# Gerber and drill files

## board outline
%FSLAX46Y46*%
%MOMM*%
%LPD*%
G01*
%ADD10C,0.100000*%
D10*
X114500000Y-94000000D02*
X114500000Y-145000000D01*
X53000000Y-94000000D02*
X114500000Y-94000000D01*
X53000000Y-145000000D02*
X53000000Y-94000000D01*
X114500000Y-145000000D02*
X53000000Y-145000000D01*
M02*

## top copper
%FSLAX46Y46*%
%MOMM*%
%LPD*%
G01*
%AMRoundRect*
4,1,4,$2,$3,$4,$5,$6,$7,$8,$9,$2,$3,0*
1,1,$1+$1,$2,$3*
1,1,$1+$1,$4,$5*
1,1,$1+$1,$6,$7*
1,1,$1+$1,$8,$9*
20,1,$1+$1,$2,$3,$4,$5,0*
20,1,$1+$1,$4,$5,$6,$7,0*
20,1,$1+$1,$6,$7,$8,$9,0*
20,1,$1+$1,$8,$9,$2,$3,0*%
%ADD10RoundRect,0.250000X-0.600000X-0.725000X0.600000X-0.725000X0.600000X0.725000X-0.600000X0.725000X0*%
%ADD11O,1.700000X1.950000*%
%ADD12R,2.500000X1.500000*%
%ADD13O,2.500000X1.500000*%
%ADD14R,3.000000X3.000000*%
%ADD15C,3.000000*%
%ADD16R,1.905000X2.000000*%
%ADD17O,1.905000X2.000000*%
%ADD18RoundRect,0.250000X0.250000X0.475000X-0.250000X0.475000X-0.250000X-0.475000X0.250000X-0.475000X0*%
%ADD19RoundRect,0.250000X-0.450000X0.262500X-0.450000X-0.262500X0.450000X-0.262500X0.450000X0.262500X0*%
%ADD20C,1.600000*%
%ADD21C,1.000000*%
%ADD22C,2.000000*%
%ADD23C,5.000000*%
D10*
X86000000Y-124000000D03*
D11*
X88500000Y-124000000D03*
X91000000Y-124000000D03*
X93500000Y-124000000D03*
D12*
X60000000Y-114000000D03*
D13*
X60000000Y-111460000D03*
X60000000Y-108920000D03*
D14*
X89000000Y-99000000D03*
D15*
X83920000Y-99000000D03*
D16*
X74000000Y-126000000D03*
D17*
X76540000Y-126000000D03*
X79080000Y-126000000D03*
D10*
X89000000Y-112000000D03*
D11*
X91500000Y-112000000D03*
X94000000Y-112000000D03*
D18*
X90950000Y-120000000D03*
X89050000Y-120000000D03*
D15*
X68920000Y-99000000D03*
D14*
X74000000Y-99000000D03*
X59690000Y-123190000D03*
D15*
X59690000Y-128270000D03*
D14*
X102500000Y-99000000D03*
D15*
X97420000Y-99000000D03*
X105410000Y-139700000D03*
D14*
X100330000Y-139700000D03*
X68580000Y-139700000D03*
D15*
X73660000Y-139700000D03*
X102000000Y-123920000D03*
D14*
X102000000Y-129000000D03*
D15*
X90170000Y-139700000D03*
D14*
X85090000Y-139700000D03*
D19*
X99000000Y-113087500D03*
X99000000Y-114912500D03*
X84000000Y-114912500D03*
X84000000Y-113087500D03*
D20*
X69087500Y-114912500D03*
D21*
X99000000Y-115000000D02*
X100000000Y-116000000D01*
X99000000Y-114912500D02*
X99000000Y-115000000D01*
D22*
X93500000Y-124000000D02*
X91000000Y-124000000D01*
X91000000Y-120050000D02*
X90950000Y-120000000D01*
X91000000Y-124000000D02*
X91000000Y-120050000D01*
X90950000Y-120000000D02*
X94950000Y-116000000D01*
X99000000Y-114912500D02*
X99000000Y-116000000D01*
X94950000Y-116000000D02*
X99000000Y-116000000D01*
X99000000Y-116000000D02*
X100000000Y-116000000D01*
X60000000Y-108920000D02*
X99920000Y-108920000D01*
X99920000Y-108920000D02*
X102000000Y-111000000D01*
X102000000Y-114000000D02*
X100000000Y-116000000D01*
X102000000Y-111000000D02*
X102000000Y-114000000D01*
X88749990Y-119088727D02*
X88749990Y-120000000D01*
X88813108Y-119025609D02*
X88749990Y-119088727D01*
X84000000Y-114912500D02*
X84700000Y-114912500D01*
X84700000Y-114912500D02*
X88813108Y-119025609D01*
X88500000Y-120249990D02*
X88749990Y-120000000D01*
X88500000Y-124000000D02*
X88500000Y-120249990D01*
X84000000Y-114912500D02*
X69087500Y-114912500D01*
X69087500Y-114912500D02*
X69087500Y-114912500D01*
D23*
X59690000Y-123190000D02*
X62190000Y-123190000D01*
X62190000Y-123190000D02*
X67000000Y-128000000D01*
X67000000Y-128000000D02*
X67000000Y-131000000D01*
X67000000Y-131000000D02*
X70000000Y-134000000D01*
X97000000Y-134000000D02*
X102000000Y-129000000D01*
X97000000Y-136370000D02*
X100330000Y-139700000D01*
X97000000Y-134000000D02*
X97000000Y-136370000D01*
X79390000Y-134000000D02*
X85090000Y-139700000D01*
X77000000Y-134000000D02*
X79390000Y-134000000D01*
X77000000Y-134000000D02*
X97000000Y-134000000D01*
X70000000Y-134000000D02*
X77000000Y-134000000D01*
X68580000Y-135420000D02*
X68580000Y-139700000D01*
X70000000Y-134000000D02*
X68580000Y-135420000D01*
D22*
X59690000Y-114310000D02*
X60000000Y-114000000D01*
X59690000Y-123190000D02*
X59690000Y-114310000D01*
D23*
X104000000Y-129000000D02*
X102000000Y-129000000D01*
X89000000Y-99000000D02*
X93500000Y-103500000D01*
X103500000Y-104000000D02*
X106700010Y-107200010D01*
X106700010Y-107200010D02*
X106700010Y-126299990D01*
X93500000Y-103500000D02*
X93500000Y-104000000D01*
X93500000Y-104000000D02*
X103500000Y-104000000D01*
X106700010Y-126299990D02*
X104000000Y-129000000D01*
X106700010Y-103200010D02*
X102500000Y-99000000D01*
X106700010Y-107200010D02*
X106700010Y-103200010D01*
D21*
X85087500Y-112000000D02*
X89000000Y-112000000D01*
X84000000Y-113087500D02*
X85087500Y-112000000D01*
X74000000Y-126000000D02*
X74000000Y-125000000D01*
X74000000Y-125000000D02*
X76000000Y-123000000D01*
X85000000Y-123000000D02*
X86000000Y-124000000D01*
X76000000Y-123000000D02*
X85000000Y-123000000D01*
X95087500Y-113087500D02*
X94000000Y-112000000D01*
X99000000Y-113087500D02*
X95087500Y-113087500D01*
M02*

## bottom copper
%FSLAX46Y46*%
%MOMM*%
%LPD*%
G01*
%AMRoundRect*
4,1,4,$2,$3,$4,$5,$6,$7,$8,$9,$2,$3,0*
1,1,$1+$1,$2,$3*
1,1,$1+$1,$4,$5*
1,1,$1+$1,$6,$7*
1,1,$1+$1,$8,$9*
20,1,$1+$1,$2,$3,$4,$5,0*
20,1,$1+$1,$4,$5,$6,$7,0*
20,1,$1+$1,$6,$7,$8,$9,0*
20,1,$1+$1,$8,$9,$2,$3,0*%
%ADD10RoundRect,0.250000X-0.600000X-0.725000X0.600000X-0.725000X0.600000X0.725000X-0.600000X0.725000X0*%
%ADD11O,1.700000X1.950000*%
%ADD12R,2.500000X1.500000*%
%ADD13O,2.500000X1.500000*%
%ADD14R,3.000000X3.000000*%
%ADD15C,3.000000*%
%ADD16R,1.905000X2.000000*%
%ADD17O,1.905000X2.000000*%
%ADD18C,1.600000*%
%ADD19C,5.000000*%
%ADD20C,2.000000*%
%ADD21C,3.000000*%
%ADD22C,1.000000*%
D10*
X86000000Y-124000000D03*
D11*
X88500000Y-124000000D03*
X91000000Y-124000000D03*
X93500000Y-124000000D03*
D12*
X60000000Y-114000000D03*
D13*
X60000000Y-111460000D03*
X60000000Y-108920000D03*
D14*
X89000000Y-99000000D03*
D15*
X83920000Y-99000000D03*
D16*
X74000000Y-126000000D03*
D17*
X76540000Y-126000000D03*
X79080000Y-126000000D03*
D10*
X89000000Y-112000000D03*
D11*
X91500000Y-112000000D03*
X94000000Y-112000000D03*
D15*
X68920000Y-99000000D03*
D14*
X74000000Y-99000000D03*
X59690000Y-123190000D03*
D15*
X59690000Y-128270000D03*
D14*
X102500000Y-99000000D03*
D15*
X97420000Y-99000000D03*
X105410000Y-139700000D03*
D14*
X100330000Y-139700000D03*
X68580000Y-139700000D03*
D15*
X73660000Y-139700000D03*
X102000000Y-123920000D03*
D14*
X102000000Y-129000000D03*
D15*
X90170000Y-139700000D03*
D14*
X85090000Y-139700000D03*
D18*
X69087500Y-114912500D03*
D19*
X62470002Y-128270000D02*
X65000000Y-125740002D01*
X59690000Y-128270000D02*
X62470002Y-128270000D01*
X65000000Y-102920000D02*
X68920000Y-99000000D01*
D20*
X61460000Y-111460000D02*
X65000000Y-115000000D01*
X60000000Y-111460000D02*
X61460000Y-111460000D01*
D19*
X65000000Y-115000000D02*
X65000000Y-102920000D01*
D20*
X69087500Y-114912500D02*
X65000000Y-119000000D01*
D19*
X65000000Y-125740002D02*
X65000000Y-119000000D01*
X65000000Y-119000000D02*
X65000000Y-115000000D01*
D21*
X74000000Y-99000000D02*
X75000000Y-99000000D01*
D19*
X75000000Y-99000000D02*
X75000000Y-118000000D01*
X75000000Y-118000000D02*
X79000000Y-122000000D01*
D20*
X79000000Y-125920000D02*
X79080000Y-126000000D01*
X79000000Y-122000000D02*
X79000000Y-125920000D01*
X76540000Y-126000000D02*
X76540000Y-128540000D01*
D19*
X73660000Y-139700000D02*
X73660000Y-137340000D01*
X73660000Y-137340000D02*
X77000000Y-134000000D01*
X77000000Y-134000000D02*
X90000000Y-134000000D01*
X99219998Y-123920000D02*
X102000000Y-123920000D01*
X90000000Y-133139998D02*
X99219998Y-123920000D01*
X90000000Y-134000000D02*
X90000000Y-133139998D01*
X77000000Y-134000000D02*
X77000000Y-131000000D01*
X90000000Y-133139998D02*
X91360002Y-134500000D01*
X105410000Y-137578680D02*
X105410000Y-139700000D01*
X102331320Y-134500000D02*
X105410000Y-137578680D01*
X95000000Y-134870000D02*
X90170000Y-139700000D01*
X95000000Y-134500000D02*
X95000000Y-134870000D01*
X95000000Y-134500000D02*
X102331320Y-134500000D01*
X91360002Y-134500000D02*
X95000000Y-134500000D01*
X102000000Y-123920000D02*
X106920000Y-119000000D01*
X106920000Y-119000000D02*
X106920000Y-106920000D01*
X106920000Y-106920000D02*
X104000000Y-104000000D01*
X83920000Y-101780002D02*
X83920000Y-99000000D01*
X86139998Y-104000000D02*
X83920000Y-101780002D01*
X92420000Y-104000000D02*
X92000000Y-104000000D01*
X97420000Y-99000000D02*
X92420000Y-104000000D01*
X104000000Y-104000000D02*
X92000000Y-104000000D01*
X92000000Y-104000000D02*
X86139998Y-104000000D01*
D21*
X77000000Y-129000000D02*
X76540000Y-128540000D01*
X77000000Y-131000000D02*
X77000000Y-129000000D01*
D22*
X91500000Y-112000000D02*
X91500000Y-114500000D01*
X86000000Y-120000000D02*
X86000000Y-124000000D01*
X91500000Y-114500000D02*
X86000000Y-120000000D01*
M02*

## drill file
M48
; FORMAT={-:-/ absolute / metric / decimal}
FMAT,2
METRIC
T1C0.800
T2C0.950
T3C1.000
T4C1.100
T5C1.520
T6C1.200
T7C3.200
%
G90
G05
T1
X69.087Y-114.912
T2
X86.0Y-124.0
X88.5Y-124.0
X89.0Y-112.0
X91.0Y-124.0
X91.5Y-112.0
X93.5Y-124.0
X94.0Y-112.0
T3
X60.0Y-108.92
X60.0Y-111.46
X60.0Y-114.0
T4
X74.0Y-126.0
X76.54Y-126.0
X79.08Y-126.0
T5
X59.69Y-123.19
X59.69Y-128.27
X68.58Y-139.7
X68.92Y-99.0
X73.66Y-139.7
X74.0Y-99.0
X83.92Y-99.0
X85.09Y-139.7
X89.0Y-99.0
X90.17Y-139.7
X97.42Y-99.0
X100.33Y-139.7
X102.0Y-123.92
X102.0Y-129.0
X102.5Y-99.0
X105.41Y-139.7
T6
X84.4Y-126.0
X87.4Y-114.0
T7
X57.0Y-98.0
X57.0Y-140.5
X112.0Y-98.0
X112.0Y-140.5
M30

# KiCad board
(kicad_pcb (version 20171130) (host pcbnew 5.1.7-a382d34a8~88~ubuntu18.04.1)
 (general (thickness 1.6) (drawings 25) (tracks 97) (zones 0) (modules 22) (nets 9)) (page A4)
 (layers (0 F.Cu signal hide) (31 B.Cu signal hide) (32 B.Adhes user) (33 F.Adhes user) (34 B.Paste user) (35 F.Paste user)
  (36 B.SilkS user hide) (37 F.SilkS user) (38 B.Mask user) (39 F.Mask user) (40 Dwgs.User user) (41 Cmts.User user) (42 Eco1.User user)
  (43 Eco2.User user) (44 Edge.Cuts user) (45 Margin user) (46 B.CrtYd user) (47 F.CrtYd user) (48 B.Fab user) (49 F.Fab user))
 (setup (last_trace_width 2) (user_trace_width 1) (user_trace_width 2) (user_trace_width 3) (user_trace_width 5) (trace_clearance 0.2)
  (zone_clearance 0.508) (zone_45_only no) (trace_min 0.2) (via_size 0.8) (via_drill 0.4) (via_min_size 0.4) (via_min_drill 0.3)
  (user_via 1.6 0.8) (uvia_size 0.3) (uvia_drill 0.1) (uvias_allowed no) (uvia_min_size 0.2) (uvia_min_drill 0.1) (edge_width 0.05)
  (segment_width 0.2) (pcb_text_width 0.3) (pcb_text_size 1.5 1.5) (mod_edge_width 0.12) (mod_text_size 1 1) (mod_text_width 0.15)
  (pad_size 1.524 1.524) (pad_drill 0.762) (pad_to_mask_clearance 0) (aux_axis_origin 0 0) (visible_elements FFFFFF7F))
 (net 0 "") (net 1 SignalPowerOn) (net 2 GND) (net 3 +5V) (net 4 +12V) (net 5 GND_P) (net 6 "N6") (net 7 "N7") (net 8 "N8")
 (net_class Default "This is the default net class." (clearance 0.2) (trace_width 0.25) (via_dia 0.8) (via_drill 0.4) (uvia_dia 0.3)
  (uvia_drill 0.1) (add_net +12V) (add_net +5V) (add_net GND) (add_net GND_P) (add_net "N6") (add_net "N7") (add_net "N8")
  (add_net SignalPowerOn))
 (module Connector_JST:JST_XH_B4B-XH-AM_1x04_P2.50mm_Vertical (layer F.Cu) (at 86 124)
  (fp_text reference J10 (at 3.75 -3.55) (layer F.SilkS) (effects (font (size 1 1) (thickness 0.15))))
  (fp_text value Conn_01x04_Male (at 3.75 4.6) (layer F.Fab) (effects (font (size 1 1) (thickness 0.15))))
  (pad 1 thru_hole roundrect (at 0 0) (size 1.7 1.95) (drill 0.95) (layers *.Cu *.Mask) (roundrect_rratio 0.147059) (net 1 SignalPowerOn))
  (pad 2 thru_hole oval (at 2.5 0) (size 1.7 1.95) (drill 0.95) (layers *.Cu *.Mask) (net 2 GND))
  (pad 3 thru_hole oval (at 5 0) (size 1.7 1.95) (drill 0.95) (layers *.Cu *.Mask) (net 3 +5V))
  (pad 4 thru_hole oval (at 7.5 0) (size 1.7 1.95) (drill 0.95) (layers *.Cu *.Mask) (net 3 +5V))
  (pad "" np_thru_hole circle (at -1.6 2) (size 1.2 1.2) (drill 1.2) (layers *.Cu *.Mask)))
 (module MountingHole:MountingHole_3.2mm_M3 (layer F.Cu) (at 57 98)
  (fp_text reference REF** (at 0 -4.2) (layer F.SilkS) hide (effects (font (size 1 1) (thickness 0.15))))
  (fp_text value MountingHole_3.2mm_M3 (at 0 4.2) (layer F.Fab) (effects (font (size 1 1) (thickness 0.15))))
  (pad 1 np_thru_hole circle (at 0 0) (size 3.2 3.2) (drill 3.2) (layers *.Cu *.Mask)))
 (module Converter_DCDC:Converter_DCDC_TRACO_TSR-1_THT (layer F.Cu) (at 60 114 90)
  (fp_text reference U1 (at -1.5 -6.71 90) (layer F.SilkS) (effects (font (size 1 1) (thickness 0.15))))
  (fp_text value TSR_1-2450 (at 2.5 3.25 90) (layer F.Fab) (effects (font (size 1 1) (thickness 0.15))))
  (pad 1 thru_hole rect (at 0 0 90) (size 1.5 2.5) (drill 1) (layers *.Cu *.Mask) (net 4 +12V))
  (pad 2 thru_hole oval (at 2.54 0 90) (size 1.5 2.5) (drill 1) (layers *.Cu *.Mask) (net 2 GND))
  (pad 3 thru_hole oval (at 5.08 0 90) (size 1.5 2.5) (drill 1) (layers *.Cu *.Mask) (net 3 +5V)))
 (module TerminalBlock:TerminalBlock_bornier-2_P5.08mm (layer F.Cu) (at 89 99 180)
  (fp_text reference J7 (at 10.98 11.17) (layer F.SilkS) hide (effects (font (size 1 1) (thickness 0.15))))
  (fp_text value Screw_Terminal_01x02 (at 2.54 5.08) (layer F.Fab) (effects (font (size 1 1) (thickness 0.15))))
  (pad 1 thru_hole rect (at 0 0 180) (size 3 3) (drill 1.52) (layers *.Cu *.Mask) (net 4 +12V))
  (pad 2 thru_hole circle (at 5.08 0 180) (size 3 3) (drill 1.52) (layers *.Cu *.Mask) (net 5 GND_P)))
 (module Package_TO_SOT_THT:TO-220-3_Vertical (layer F.Cu) (at 74 126)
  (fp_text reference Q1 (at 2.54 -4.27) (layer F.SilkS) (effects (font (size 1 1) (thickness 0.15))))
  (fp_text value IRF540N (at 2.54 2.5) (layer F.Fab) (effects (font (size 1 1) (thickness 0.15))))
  (pad 1 thru_hole rect (at 0 0) (size 1.905 2) (drill 1.1) (layers *.Cu *.Mask) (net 1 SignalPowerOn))
  (pad 2 thru_hole oval (at 2.54 0) (size 1.905 2) (drill 1.1) (layers *.Cu *.Mask) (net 5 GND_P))
  (pad 3 thru_hole oval (at 5.08 0) (size 1.905 2) (drill 1.1) (layers *.Cu *.Mask) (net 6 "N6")))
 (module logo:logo (layer B.Cu) (at 78 111.5)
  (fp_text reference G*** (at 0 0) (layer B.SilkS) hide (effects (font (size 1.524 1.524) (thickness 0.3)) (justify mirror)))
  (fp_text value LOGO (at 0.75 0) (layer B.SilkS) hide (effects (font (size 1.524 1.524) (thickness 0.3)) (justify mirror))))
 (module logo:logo (layer F.Cu) (at 69 -16)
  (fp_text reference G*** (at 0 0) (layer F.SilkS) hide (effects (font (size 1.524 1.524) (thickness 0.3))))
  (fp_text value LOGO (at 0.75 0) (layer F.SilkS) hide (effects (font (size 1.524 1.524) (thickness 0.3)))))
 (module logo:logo (layer F.Cu) (at 94 104)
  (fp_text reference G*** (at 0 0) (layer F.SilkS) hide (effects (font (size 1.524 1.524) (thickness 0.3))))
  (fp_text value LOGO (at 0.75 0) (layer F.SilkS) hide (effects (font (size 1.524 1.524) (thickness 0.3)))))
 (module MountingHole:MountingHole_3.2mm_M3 (layer F.Cu) (at 57 140.5)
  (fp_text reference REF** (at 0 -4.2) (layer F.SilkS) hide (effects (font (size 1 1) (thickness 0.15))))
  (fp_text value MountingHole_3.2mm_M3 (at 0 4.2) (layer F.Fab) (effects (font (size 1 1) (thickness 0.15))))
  (pad 1 np_thru_hole circle (at 0 0) (size 3.2 3.2) (drill 3.2) (layers *.Cu *.Mask)))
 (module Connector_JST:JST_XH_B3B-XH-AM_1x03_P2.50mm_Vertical (layer F.Cu) (at 89 112)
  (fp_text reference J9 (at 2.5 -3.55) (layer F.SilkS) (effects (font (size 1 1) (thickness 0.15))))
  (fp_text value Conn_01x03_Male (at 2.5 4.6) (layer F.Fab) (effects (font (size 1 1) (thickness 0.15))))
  (pad 1 thru_hole roundrect (at 0 0) (size 1.7 1.95) (drill 0.95) (layers *.Cu *.Mask) (roundrect_rratio 0.147059) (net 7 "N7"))
  (pad 2 thru_hole oval (at 2.5 0) (size 1.7 1.95) (drill 0.95) (layers *.Cu *.Mask) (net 1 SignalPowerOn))
  (pad 3 thru_hole oval (at 5 0) (size 1.7 1.95) (drill 0.95) (layers *.Cu *.Mask) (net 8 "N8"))
  (pad "" np_thru_hole circle (at -1.6 2) (size 1.2 1.2) (drill 1.2) (layers *.Cu *.Mask)))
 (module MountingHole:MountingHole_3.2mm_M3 (layer F.Cu) (at 112 98)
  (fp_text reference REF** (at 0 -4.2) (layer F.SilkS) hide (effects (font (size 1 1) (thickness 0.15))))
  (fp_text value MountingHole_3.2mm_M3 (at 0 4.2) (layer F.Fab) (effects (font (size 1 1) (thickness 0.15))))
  (pad 1 np_thru_hole circle (at 0 0) (size 3.2 3.2) (drill 3.2) (layers *.Cu *.Mask)))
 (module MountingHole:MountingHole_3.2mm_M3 (layer F.Cu) (at 112 140.5)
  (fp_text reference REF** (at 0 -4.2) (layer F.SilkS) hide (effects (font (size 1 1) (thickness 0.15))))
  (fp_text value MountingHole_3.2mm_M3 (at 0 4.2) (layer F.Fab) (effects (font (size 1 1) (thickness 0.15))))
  (pad 1 np_thru_hole circle (at 0 0) (size 3.2 3.2) (drill 3.2) (layers *.Cu *.Mask)))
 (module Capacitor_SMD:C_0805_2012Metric (layer F.Cu) (at 90 120 180)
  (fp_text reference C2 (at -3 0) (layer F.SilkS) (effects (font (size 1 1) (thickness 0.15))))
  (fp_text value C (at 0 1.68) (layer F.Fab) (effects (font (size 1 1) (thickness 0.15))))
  (pad 1 smd roundrect (at -0.95 0 180) (size 1 1.45) (layers F.Cu F.Paste F.Mask) (roundrect_rratio 0.25) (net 3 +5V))
  (pad 2 smd roundrect (at 0.95 0 180) (size 1 1.45) (layers F.Cu F.Paste F.Mask) (roundrect_rratio 0.25) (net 2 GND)))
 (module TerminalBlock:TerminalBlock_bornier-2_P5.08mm (layer F.Cu) (at 74 99 180)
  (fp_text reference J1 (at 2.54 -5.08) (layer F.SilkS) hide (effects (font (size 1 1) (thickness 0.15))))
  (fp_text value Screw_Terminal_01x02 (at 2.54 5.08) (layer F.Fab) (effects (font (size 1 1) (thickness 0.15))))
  (pad 2 thru_hole circle (at 5.08 0 180) (size 3 3) (drill 1.52) (layers *.Cu *.Mask) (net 2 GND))
  (pad 1 thru_hole rect (at 0 0 180) (size 3 3) (drill 1.52) (layers *.Cu *.Mask) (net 6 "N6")))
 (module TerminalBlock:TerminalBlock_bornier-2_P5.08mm (layer F.Cu) (at 59.69 123.19 270)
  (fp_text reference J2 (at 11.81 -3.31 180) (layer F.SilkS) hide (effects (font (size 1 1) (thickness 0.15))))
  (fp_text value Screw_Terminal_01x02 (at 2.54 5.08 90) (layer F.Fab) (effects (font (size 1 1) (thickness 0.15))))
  (pad 1 thru_hole rect (at 0 0 270) (size 3 3) (drill 1.52) (layers *.Cu *.Mask) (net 4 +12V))
  (pad 2 thru_hole circle (at 5.08 0 270) (size 3 3) (drill 1.52) (layers *.Cu *.Mask) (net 2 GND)))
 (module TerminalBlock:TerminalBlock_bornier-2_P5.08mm (layer F.Cu) (at 102.5 99 180)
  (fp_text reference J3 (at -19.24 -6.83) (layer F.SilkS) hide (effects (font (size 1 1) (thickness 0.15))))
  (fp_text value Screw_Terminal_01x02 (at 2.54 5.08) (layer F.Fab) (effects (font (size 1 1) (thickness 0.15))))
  (pad 1 thru_hole rect (at 0 0 180) (size 3 3) (drill 1.52) (layers *.Cu *.Mask) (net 4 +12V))
  (pad 2 thru_hole circle (at 5.08 0 180) (size 3 3) (drill 1.52) (layers *.Cu *.Mask) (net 5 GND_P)))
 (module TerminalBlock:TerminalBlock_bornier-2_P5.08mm (layer F.Cu) (at 100.33 139.7)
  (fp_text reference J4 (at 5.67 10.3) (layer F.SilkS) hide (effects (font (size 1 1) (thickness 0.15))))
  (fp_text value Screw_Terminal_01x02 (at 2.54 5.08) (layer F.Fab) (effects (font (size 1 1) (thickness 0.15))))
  (pad 2 thru_hole circle (at 5.08 0) (size 3 3) (drill 1.52) (layers *.Cu *.Mask) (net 5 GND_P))
  (pad 1 thru_hole rect (at 0 0) (size 3 3) (drill 1.52) (layers *.Cu *.Mask) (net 4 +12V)))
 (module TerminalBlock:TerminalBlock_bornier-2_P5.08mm (layer F.Cu) (at 68.58 139.7)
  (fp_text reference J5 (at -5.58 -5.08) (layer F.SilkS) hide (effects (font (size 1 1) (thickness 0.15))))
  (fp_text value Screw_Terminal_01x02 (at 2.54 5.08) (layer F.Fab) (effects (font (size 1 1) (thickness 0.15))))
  (pad 1 thru_hole rect (at 0 0) (size 3 3) (drill 1.52) (layers *.Cu *.Mask) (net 4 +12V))
  (pad 2 thru_hole circle (at 5.08 0) (size 3 3) (drill 1.52) (layers *.Cu *.Mask) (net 5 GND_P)))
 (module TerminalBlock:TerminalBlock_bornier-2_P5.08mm (layer F.Cu) (at 102 129 90)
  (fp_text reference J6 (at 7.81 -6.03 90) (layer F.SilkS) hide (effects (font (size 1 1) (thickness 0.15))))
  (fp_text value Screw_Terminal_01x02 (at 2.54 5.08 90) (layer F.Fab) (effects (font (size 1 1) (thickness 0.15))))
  (pad 2 thru_hole circle (at 5.08 0 90) (size 3 3) (drill 1.52) (layers *.Cu *.Mask) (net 5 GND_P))
  (pad 1 thru_hole rect (at 0 0 90) (size 3 3) (drill 1.52) (layers *.Cu *.Mask) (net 4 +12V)))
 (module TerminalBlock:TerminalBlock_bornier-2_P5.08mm (layer F.Cu) (at 85.09 139.7)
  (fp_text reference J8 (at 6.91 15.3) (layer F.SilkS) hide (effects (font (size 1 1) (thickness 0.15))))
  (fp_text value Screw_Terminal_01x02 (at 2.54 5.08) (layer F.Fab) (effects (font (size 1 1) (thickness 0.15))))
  (pad 2 thru_hole circle (at 5.08 0) (size 3 3) (drill 1.52) (layers *.Cu *.Mask) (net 5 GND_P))
  (pad 1 thru_hole rect (at 0 0) (size 3 3) (drill 1.52) (layers *.Cu *.Mask) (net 4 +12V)))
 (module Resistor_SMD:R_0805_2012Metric (layer F.Cu) (at 99 114 270)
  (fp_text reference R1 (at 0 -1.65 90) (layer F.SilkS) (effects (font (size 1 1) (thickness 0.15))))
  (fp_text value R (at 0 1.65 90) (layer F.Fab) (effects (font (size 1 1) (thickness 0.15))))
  (pad 1 smd roundrect (at -0.9125 0 270) (size 1.025 1.4) (layers F.Cu F.Paste F.Mask) (roundrect_rratio 0.243902) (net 8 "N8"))
  (pad 2 smd roundrect (at 0.9125 0 270) (size 1.025 1.4) (layers F.Cu F.Paste F.Mask) (roundrect_rratio 0.243902) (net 3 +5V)))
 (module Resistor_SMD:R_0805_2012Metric (layer F.Cu) (at 84 114 270)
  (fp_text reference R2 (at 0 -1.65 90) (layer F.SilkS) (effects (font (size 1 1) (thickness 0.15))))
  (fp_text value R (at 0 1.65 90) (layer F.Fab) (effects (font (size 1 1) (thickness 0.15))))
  (pad 2 smd roundrect (at 0.9125 0 270) (size 1.025 1.4) (layers F.Cu F.Paste F.Mask) (roundrect_rratio 0.243902) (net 2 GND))
  (pad 1 smd roundrect (at -0.9125 0 270) (size 1.025 1.4) (layers F.Cu F.Paste F.Mask) (roundrect_rratio 0.243902) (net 7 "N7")))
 (gr_line (start 114.5 94) (end 114.5 145) (layer Edge.Cuts) (width 0.1))
 (gr_line (start 53 94) (end 114.5 94) (layer Edge.Cuts) (width 0.1))
 (gr_line (start 53 145) (end 53 94) (layer Edge.Cuts) (width 0.1))
 (gr_line (start 114.5 145) (end 53 145) (layer Edge.Cuts) (width 0.1))
 (segment (start 99 115) (end 100 116) (width 1) (layer F.Cu) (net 3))
 (segment (start 99 114.9125) (end 99 115) (width 1) (layer F.Cu) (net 3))
 (segment (start 93.5 124) (end 91 124) (width 2) (layer F.Cu) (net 3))
 (segment (start 91 120.05) (end 90.95 120) (width 2) (layer F.Cu) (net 3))
 (segment (start 91 124) (end 91 120.05) (width 2) (layer F.Cu) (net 3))
 (segment (start 90.95 120) (end 94.95 116) (width 2) (layer F.Cu) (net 3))
 (segment (start 99 114.9125) (end 99 116) (width 2) (layer F.Cu) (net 3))
 (segment (start 94.95 116) (end 99 116) (width 2) (layer F.Cu) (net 3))
 (segment (start 99 116) (end 100 116) (width 2) (layer F.Cu) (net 3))
 (segment (start 60 108.92) (end 99.92 108.92) (width 2) (layer F.Cu) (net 3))
 (segment (start 99.92 108.92) (end 102 111) (width 2) (layer F.Cu) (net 3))
 (segment (start 102 114) (end 100 116) (width 2) (layer F.Cu) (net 3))
 (segment (start 102 111) (end 102 114) (width 2) (layer F.Cu) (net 3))
 (segment (start 62.470002 128.27) (end 65 125.740002) (width 5) (layer B.Cu) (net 2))
 (segment (start 59.69 128.27) (end 62.470002 128.27) (width 5) (layer B.Cu) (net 2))
 (segment (start 65 102.92) (end 68.92 99) (width 5) (layer B.Cu) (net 2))
 (segment (start 61.46 111.46) (end 65 115) (width 2) (layer B.Cu) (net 2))
 (segment (start 60 111.46) (end 61.46 111.46) (width 2) (layer B.Cu) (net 2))
 (segment (start 65 115) (end 65 102.92) (width 5) (layer B.Cu) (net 2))
 (segment (start 88.74999 119.088727) (end 88.74999 120) (width 2) (layer F.Cu) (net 2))
 (segment (start 88.813108 119.025609) (end 88.74999 119.088727) (width 2) (layer F.Cu) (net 2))
 (segment (start 84 114.9125) (end 84.7 114.9125) (width 2) (layer F.Cu) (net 2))
 (segment (start 84.7 114.9125) (end 88.813108 119.025609) (width 2) (layer F.Cu) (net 2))
 (segment (start 88.5 120.24999) (end 88.74999 120) (width 2) (layer F.Cu) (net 2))
 (segment (start 88.5 124) (end 88.5 120.24999) (width 2) (layer F.Cu) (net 2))
 (segment (start 84 114.9125) (end 69.0875 114.9125) (width 2) (layer F.Cu) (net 2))
 (segment (start 69.0875 114.9125) (end 69.0875 114.9125) (width 2) (layer F.Cu) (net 2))
 (via (at 69.0875 114.9125) (size 1.6) (drill 0.8) (layers F.Cu B.Cu) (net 2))
 (segment (start 69.0875 114.9125) (end 65 119) (width 2) (layer B.Cu) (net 2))
 (segment (start 65 125.740002) (end 65 119) (width 5) (layer B.Cu) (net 2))
 (segment (start 65 119) (end 65 115) (width 5) (layer B.Cu) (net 2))
 (segment (start 74 99) (end 75 99) (width 3) (layer B.Cu) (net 6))
 (segment (start 75 99) (end 75 118) (width 5) (layer B.Cu) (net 6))
 (segment (start 75 118) (end 79 122) (width 5) (layer B.Cu) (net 6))
 (segment (start 79 125.92) (end 79.08 126) (width 2) (layer B.Cu) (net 6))
 (segment (start 79 122) (end 79 125.92) (width 2) (layer B.Cu) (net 6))
 (segment (start 59.69 123.19) (end 62.19 123.19) (width 5) (layer F.Cu) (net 4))
 (segment (start 62.19 123.19) (end 67 128) (width 5) (layer F.Cu) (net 4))
 (segment (start 67 128) (end 67 131) (width 5) (layer F.Cu) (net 4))
 (segment (start 67 131) (end 70 134) (width 5) (layer F.Cu) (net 4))
 (segment (start 97 134) (end 102 129) (width 5) (layer F.Cu) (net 4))
 (segment (start 97 136.37) (end 100.33 139.7) (width 5) (layer F.Cu) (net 4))
 (segment (start 97 134) (end 97 136.37) (width 5) (layer F.Cu) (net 4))
 (segment (start 79.39 134) (end 85.09 139.7) (width 5) (layer F.Cu) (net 4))
 (segment (start 77 134) (end 79.39 134) (width 5) (layer F.Cu) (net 4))
 (segment (start 77 134) (end 97 134) (width 5) (layer F.Cu) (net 4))
 (segment (start 70 134) (end 77 134) (width 5) (layer F.Cu) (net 4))
 (segment (start 68.58 135.42) (end 68.58 139.7) (width 5) (layer F.Cu) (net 4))
 (segment (start 70 134) (end 68.58 135.42) (width 5) (layer F.Cu) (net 4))
 (segment (start 59.69 114.31) (end 60 114) (width 2) (layer F.Cu) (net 4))
 (segment (start 59.69 123.19) (end 59.69 114.31) (width 2) (layer F.Cu) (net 4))
 (segment (start 104 129) (end 102 129) (width 5) (layer F.Cu) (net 4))
 (segment (start 89 99) (end 93.5 103.5) (width 5) (layer F.Cu) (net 4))
 (segment (start 103.5 104) (end 106.70001 107.20001) (width 5) (layer F.Cu) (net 4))
 (segment (start 106.70001 107.20001) (end 106.70001 126.29999) (width 5) (layer F.Cu) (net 4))
 (segment (start 93.5 103.5) (end 93.5 104) (width 5) (layer F.Cu) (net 4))
 (segment (start 93.5 104) (end 103.5 104) (width 5) (layer F.Cu) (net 4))
 (segment (start 106.70001 126.29999) (end 104 129) (width 5) (layer F.Cu) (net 4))
 (segment (start 106.70001 103.20001) (end 102.5 99) (width 5) (layer F.Cu) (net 4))
 (segment (start 106.70001 107.20001) (end 106.70001 103.20001) (width 5) (layer F.Cu) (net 4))
 (segment (start 76.54 126) (end 76.54 128.54) (width 2) (layer B.Cu) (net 5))
 (segment (start 73.66 139.7) (end 73.66 137.34) (width 5) (layer B.Cu) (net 5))
 (segment (start 73.66 137.34) (end 77 134) (width 5) (layer B.Cu) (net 5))
 (segment (start 77 134) (end 90 134) (width 5) (layer B.Cu) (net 5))
 (segment (start 99.219998 123.92) (end 102 123.92) (width 5) (layer B.Cu) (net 5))
 (segment (start 90 133.139998) (end 99.219998 123.92) (width 5) (layer B.Cu) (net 5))
 (segment (start 90 134) (end 90 133.139998) (width 5) (layer B.Cu) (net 5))
 (segment (start 77 134) (end 77 131) (width 5) (layer B.Cu) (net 5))
 (segment (start 90 133.139998) (end 91.360002 134.5) (width 5) (layer B.Cu) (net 5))
 (segment (start 105.41 137.57868) (end 105.41 139.7) (width 5) (layer B.Cu) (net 5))
 (segment (start 102.33132 134.5) (end 105.41 137.57868) (width 5) (layer B.Cu) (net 5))
 (segment (start 95 134.87) (end 90.17 139.7) (width 5) (layer B.Cu) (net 5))
 (segment (start 95 134.5) (end 95 134.87) (width 5) (layer B.Cu) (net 5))
 (segment (start 95 134.5) (end 102.33132 134.5) (width 5) (layer B.Cu) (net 5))
 (segment (start 91.360002 134.5) (end 95 134.5) (width 5) (layer B.Cu) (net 5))
 (segment (start 102 123.92) (end 106.92 119) (width 5) (layer B.Cu) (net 5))
 (segment (start 106.92 119) (end 106.92 106.92) (width 5) (layer B.Cu) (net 5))
 (segment (start 106.92 106.92) (end 104 104) (width 5) (layer B.Cu) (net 5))
 (segment (start 83.92 101.780002) (end 83.92 99) (width 5) (layer B.Cu) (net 5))
 (segment (start 86.139998 104) (end 83.92 101.780002) (width 5) (layer B.Cu) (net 5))
 (segment (start 92.42 104) (end 92 104) (width 5) (layer B.Cu) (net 5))
 (segment (start 97.42 99) (end 92.42 104) (width 5) (layer B.Cu) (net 5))
 (segment (start 104 104) (end 92 104) (width 5) (layer B.Cu) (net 5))
 (segment (start 92 104) (end 86.139998 104) (width 5) (layer B.Cu) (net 5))
 (segment (start 77 129) (end 76.54 128.54) (width 3) (layer B.Cu) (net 5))
 (segment (start 77 131) (end 77 129) (width 3) (layer B.Cu) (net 5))
 (segment (start 85.0875 112) (end 89 112) (width 1) (layer F.Cu) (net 7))
 (segment (start 84 113.0875) (end 85.0875 112) (width 1) (layer F.Cu) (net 7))
 (segment (start 74 126) (end 74 125) (width 1) (layer F.Cu) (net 1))
 (segment (start 74 125) (end 76 123) (width 1) (layer F.Cu) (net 1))
 (segment (start 85 123) (end 86 124) (width 1) (layer F.Cu) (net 1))
 (segment (start 76 123) (end 85 123) (width 1) (layer F.Cu) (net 1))
 (segment (start 91.5 112) (end 91.5 114.5) (width 1) (layer B.Cu) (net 1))
 (segment (start 86 120) (end 86 124) (width 1) (layer B.Cu) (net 1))
 (segment (start 91.5 114.5) (end 86 120) (width 1) (layer B.Cu) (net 1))
 (segment (start 95.0875 113.0875) (end 94 112) (width 1) (layer F.Cu) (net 8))
 (segment (start 99 113.0875) (end 95.0875 113.0875) (width 1) (layer F.Cu) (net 8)))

